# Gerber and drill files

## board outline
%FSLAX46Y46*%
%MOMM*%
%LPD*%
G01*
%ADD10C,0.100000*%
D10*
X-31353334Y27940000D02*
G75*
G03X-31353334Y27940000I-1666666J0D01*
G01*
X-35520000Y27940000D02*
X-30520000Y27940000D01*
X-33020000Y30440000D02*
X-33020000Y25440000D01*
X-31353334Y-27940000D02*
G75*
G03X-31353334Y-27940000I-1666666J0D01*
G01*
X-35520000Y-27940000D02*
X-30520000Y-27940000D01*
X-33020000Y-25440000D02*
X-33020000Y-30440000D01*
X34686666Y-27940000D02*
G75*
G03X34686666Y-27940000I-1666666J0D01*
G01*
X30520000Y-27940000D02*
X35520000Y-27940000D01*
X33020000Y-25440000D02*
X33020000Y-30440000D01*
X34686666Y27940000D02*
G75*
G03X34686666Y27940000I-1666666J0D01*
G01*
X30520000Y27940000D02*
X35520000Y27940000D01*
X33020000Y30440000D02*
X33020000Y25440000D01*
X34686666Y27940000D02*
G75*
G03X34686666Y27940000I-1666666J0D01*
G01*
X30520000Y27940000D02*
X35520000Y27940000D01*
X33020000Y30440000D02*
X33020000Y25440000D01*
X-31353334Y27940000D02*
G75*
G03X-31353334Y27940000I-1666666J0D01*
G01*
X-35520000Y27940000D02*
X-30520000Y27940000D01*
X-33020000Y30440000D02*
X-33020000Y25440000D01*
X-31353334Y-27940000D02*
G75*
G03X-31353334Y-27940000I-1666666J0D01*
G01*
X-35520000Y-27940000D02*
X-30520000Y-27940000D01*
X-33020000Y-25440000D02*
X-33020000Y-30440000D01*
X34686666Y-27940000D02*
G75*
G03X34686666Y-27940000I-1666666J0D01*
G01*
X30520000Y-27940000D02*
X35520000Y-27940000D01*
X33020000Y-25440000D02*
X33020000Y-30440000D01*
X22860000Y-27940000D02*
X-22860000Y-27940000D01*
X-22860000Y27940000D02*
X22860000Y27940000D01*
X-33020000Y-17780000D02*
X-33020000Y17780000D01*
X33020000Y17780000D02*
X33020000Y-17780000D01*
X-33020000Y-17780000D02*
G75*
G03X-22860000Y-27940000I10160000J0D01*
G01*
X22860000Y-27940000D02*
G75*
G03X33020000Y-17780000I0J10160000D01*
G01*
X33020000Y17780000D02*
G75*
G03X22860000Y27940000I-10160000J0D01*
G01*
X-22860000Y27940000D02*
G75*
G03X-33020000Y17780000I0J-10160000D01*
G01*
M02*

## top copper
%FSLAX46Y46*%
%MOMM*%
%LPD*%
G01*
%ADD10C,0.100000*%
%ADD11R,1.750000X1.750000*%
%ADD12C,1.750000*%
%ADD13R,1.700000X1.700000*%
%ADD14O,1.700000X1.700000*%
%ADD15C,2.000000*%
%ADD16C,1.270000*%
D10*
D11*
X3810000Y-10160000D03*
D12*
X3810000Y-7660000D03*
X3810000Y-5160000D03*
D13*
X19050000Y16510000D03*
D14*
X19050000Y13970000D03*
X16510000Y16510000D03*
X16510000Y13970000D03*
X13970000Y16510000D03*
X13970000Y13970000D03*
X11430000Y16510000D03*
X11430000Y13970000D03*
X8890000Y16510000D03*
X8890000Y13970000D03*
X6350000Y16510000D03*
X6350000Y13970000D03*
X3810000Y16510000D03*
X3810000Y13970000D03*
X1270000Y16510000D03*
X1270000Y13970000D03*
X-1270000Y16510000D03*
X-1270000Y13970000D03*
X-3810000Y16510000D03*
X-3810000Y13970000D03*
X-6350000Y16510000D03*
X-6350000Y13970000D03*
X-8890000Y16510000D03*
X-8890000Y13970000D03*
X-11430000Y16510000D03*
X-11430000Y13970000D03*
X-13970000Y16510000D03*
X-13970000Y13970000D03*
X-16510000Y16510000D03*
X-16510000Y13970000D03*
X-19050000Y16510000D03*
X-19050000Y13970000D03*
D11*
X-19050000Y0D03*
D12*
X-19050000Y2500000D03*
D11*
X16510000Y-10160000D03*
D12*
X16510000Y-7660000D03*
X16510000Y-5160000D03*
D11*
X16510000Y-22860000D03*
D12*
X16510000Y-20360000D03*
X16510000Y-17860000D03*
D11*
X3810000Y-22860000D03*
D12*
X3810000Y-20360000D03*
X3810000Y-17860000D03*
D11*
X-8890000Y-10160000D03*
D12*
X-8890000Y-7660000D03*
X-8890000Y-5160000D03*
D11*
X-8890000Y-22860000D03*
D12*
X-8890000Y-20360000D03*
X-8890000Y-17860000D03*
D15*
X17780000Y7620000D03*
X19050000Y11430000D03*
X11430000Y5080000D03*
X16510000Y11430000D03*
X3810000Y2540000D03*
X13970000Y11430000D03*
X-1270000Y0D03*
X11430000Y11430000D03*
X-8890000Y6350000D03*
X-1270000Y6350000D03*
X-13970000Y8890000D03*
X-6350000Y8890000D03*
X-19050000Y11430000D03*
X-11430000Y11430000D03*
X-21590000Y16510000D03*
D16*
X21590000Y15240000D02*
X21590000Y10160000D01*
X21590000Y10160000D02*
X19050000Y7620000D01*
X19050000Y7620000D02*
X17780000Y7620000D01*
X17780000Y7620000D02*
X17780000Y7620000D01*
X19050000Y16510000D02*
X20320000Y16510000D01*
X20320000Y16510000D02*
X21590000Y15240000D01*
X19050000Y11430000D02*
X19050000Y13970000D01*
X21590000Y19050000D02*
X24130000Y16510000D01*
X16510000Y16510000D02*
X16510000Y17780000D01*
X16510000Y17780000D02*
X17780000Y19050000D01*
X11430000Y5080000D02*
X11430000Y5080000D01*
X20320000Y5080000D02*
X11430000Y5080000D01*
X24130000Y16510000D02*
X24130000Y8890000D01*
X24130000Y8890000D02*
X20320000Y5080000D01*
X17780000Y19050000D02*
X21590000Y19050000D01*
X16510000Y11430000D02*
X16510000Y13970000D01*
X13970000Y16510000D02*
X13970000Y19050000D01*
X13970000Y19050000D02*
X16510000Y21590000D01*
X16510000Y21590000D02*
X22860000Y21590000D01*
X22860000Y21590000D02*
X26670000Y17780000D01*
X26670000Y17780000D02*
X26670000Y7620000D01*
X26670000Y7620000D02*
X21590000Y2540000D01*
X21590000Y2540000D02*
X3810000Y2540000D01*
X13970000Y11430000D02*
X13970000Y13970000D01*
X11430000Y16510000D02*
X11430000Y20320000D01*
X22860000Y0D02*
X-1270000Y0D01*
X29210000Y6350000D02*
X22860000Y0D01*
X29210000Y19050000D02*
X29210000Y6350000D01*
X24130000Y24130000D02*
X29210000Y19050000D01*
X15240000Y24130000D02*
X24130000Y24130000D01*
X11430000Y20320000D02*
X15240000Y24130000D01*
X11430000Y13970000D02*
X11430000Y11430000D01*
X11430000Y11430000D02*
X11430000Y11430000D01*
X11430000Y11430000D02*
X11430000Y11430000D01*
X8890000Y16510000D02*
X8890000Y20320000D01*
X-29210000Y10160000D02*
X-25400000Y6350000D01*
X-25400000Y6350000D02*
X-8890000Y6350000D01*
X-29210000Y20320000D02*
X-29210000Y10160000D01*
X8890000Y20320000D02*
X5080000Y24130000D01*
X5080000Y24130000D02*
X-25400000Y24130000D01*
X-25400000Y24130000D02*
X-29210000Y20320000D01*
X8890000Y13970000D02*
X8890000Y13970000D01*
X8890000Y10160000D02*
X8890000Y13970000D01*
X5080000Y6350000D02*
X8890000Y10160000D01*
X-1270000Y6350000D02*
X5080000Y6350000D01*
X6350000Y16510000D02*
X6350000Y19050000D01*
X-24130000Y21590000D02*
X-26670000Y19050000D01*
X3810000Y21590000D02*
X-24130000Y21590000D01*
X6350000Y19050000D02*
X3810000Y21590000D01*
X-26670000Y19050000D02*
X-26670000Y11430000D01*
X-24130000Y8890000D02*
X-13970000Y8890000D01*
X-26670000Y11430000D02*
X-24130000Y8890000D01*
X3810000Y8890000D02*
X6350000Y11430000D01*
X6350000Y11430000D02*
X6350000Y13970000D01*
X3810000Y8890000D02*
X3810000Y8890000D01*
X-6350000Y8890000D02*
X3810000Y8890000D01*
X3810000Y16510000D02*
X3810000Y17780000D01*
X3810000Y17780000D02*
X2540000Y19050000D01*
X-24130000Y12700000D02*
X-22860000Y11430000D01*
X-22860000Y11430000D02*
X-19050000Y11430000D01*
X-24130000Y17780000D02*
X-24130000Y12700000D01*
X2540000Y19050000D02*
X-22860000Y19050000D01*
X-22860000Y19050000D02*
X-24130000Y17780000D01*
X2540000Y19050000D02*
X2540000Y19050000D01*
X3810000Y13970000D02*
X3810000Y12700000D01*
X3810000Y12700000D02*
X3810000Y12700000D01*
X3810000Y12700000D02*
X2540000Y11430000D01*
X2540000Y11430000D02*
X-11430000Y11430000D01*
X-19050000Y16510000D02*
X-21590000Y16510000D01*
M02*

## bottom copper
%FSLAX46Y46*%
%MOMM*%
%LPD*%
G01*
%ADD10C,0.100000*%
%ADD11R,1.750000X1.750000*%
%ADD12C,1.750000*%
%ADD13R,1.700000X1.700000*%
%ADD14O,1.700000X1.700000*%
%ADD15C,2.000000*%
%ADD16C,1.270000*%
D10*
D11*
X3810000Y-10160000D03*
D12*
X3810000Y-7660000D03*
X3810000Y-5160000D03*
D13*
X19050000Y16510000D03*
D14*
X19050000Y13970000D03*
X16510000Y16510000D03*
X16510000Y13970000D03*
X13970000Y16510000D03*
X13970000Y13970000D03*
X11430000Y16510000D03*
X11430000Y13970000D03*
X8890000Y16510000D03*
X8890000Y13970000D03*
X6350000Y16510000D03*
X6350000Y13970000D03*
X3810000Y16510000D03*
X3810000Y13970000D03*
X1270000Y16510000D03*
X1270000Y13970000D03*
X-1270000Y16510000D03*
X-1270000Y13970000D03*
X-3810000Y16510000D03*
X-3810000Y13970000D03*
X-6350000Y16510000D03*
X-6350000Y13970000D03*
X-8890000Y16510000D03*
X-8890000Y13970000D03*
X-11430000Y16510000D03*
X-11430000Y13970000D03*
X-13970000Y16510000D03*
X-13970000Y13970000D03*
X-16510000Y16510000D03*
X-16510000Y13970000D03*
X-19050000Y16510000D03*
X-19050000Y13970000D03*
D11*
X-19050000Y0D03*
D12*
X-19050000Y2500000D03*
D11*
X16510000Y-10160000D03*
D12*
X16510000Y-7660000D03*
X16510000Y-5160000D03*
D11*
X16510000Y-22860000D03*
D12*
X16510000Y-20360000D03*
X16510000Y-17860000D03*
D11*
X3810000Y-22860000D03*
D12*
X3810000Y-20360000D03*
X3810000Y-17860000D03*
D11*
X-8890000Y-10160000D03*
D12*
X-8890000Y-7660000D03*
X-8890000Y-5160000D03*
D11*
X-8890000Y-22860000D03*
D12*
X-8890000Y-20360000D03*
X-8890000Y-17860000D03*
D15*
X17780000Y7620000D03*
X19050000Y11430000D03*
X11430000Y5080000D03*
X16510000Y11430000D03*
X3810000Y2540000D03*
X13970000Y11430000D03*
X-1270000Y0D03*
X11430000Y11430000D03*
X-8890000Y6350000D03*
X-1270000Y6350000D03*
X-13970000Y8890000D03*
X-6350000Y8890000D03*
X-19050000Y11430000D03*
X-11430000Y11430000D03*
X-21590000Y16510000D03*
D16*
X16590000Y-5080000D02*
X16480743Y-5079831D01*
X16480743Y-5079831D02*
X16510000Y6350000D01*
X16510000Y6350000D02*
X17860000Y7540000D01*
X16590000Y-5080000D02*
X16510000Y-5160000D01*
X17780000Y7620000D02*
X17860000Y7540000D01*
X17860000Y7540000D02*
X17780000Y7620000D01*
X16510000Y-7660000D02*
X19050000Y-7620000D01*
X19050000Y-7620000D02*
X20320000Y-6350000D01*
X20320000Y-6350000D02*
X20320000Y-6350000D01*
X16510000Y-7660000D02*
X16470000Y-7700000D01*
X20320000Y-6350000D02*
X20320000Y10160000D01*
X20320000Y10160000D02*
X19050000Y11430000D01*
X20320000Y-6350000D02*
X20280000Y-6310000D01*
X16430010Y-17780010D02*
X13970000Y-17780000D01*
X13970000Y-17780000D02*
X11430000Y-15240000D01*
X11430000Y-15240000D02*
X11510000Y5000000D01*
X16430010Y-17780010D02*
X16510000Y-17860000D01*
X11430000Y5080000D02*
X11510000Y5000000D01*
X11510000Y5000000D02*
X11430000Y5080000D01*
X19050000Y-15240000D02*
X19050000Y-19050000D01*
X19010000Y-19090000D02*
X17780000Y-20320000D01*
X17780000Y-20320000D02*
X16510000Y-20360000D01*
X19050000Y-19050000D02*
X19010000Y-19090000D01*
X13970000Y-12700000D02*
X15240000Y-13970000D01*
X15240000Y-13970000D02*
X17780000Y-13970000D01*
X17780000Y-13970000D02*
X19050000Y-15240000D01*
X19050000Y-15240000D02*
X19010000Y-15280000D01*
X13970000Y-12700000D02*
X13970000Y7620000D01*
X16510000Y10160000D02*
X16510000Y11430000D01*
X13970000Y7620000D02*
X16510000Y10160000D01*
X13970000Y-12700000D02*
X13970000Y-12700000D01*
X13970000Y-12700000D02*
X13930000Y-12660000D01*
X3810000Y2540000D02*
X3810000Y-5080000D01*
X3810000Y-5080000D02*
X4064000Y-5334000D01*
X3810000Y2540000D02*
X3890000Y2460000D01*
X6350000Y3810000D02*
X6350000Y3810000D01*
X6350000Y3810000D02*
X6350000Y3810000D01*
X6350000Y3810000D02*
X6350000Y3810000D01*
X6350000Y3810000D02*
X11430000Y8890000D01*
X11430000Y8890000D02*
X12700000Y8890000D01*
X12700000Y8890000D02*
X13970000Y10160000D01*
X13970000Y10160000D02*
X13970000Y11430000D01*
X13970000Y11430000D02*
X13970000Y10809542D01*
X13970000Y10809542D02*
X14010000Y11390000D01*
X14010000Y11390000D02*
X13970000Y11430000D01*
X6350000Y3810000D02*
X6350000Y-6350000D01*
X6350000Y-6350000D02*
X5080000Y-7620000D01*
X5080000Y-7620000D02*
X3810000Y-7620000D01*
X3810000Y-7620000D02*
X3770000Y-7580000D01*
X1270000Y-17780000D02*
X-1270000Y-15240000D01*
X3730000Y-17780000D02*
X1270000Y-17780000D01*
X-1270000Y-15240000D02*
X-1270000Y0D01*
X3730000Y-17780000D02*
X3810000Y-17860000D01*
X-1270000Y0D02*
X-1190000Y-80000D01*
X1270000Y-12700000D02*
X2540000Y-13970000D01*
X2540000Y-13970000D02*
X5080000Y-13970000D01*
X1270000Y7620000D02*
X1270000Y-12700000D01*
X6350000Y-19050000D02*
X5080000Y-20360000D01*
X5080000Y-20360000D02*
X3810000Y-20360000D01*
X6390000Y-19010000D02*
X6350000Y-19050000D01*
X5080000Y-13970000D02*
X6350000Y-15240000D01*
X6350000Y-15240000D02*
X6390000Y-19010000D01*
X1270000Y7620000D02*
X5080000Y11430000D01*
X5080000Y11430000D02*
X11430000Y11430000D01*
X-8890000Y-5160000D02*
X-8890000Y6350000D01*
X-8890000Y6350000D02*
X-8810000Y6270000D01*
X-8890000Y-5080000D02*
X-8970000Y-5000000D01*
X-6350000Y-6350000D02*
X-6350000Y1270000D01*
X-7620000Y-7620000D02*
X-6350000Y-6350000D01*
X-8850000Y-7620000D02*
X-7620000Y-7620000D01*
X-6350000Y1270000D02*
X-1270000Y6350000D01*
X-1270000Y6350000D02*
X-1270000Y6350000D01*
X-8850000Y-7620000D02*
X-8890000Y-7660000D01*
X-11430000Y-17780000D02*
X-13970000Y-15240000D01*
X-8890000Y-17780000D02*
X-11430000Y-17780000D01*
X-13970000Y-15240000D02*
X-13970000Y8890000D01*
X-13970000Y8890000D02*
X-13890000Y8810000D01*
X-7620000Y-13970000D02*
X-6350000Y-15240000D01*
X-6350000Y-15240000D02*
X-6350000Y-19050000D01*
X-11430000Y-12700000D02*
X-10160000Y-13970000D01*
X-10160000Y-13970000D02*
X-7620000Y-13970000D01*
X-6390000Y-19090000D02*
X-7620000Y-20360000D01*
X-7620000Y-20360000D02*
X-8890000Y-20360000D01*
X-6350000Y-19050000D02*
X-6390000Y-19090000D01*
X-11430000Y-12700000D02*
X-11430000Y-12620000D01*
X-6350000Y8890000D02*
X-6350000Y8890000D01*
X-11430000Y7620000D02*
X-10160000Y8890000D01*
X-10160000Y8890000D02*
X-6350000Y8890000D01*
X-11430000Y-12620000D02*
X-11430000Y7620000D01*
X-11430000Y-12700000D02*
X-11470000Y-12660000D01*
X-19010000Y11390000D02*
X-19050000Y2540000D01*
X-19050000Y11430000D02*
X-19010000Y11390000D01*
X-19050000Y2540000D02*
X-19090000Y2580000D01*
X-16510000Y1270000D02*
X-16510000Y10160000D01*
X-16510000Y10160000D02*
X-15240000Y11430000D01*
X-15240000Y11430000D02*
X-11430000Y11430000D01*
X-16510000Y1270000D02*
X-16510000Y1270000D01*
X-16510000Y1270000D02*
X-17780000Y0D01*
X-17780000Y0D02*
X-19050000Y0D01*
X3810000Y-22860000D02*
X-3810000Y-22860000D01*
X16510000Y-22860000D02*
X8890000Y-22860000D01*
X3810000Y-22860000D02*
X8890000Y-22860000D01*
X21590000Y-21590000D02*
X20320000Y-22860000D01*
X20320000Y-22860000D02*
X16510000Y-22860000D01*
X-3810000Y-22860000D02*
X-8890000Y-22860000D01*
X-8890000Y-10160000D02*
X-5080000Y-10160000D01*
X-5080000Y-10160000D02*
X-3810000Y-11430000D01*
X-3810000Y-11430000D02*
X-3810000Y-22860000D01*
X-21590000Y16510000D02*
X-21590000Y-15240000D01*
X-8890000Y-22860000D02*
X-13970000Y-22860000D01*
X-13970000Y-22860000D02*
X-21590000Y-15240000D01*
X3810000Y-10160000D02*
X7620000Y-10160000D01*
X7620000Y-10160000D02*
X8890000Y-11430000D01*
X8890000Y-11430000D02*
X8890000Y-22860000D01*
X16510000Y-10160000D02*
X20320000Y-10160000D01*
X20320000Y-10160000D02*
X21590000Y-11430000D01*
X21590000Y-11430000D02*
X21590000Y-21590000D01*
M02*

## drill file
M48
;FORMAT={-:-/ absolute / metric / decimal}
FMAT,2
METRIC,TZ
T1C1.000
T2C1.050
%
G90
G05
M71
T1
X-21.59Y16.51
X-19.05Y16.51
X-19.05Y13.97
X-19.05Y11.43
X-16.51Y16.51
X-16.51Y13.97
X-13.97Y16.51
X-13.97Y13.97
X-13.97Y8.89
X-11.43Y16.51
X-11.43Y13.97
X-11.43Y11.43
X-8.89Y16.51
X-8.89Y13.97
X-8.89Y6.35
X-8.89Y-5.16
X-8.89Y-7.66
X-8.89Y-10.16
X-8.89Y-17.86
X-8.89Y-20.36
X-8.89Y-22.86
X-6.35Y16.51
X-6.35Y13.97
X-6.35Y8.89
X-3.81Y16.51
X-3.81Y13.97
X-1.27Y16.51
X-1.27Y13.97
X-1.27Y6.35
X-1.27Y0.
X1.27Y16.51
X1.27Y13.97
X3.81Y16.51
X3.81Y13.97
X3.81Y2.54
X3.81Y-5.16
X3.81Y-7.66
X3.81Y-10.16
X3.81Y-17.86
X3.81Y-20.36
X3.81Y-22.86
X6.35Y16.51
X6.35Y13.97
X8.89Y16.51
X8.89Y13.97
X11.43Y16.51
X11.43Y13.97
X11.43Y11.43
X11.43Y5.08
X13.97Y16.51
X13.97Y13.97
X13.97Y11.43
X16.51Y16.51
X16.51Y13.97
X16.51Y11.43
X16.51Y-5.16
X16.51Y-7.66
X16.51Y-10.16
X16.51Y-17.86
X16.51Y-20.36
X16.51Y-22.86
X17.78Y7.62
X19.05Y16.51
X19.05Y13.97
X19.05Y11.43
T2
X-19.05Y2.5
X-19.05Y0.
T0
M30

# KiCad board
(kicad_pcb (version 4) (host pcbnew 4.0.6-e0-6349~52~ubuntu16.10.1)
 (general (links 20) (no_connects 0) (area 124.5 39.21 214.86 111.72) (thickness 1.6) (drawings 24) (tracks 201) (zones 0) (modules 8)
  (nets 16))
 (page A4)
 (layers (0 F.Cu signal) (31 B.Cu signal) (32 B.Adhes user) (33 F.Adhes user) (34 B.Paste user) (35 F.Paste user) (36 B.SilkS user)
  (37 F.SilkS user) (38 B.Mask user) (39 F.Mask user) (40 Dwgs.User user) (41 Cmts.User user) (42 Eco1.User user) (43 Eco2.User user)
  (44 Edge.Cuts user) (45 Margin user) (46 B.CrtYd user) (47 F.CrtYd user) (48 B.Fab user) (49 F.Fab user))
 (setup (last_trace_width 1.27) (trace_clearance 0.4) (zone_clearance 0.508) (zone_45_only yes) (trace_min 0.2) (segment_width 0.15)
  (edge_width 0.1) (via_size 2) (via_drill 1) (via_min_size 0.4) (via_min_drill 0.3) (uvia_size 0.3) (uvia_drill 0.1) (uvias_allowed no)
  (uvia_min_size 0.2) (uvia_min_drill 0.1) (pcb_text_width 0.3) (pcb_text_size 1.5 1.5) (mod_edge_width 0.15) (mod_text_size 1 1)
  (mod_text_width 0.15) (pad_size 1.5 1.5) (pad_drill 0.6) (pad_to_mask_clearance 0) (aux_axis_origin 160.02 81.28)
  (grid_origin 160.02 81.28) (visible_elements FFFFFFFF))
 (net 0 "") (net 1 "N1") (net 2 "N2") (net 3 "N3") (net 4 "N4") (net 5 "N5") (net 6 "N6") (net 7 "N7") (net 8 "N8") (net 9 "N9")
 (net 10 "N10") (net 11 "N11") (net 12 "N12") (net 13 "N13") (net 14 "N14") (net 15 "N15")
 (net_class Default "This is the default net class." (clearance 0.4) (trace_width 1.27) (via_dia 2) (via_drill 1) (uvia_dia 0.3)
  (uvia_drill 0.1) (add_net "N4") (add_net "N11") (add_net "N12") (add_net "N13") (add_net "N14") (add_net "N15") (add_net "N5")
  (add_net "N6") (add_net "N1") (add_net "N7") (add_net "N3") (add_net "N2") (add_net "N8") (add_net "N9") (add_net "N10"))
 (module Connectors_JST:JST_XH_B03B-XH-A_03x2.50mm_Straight (layer F.Cu) (at 163.83 91.44 90)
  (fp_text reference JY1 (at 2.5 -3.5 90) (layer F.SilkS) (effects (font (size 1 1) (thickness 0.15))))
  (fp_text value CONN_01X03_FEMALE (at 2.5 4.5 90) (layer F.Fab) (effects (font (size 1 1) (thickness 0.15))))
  (pad 1 thru_hole rect (at 0 0 90) (size 1.75 1.75) (drill 1) (layers *.Cu *.Mask) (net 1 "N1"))
  (pad 2 thru_hole circle (at 2.5 0 90) (size 1.75 1.75) (drill 1) (layers *.Cu *.Mask) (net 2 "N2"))
  (pad 3 thru_hole circle (at 5 0 90) (size 1.75 1.75) (drill 1) (layers *.Cu *.Mask) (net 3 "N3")))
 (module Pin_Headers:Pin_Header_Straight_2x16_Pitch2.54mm (layer F.Cu) (at 179.07 64.77 270)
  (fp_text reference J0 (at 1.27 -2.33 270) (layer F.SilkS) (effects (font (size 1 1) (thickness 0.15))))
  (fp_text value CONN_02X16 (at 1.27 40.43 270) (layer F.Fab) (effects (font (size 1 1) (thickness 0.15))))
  (pad 1 thru_hole rect (at 0 0 270) (size 1.7 1.7) (drill 1) (layers *.Cu *.Mask) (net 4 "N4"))
  (pad 2 thru_hole oval (at 2.54 0 270) (size 1.7 1.7) (drill 1) (layers *.Cu *.Mask) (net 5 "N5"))
  (pad 3 thru_hole oval (at 0 2.54 270) (size 1.7 1.7) (drill 1) (layers *.Cu *.Mask) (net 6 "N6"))
  (pad 4 thru_hole oval (at 2.54 2.54 270) (size 1.7 1.7) (drill 1) (layers *.Cu *.Mask) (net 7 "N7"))
  (pad 5 thru_hole oval (at 0 5.08 270) (size 1.7 1.7) (drill 1) (layers *.Cu *.Mask) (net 3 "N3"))
  (pad 6 thru_hole oval (at 2.54 5.08 270) (size 1.7 1.7) (drill 1) (layers *.Cu *.Mask) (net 2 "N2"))
  (pad 7 thru_hole oval (at 0 7.62 270) (size 1.7 1.7) (drill 1) (layers *.Cu *.Mask) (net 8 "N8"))
  (pad 8 thru_hole oval (at 2.54 7.62 270) (size 1.7 1.7) (drill 1) (layers *.Cu *.Mask) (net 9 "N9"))
  (pad 9 thru_hole oval (at 0 10.16 270) (size 1.7 1.7) (drill 1) (layers *.Cu *.Mask) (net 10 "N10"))
  (pad 10 thru_hole oval (at 2.54 10.16 270) (size 1.7 1.7) (drill 1) (layers *.Cu *.Mask) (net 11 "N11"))
  (pad 11 thru_hole oval (at 0 12.7 270) (size 1.7 1.7) (drill 1) (layers *.Cu *.Mask) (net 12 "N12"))
  (pad 12 thru_hole oval (at 2.54 12.7 270) (size 1.7 1.7) (drill 1) (layers *.Cu *.Mask) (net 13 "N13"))
  (pad 13 thru_hole oval (at 0 15.24 270) (size 1.7 1.7) (drill 1) (layers *.Cu *.Mask) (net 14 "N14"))
  (pad 14 thru_hole oval (at 2.54 15.24 270) (size 1.7 1.7) (drill 1) (layers *.Cu *.Mask) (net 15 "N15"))
  (pad 15 thru_hole oval (at 0 17.78 270) (size 1.7 1.7) (drill 1) (layers *.Cu *.Mask))
  (pad 16 thru_hole oval (at 2.54 17.78 270) (size 1.7 1.7) (drill 1) (layers *.Cu *.Mask))
  (pad 17 thru_hole oval (at 0 20.32 270) (size 1.7 1.7) (drill 1) (layers *.Cu *.Mask))
  (pad 18 thru_hole oval (at 2.54 20.32 270) (size 1.7 1.7) (drill 1) (layers *.Cu *.Mask))
  (pad 19 thru_hole oval (at 0 22.86 270) (size 1.7 1.7) (drill 1) (layers *.Cu *.Mask))
  (pad 20 thru_hole oval (at 2.54 22.86 270) (size 1.7 1.7) (drill 1) (layers *.Cu *.Mask))
  (pad 21 thru_hole oval (at 0 25.4 270) (size 1.7 1.7) (drill 1) (layers *.Cu *.Mask))
  (pad 22 thru_hole oval (at 2.54 25.4 270) (size 1.7 1.7) (drill 1) (layers *.Cu *.Mask))
  (pad 23 thru_hole oval (at 0 27.94 270) (size 1.7 1.7) (drill 1) (layers *.Cu *.Mask))
  (pad 24 thru_hole oval (at 2.54 27.94 270) (size 1.7 1.7) (drill 1) (layers *.Cu *.Mask))
  (pad 25 thru_hole oval (at 0 30.48 270) (size 1.7 1.7) (drill 1) (layers *.Cu *.Mask))
  (pad 26 thru_hole oval (at 2.54 30.48 270) (size 1.7 1.7) (drill 1) (layers *.Cu *.Mask))
  (pad 27 thru_hole oval (at 0 33.02 270) (size 1.7 1.7) (drill 1) (layers *.Cu *.Mask))
  (pad 28 thru_hole oval (at 2.54 33.02 270) (size 1.7 1.7) (drill 1) (layers *.Cu *.Mask))
  (pad 29 thru_hole oval (at 0 35.56 270) (size 1.7 1.7) (drill 1) (layers *.Cu *.Mask))
  (pad 30 thru_hole oval (at 2.54 35.56 270) (size 1.7 1.7) (drill 1) (layers *.Cu *.Mask))
  (pad 31 thru_hole oval (at 0 38.1 270) (size 1.7 1.7) (drill 1) (layers *.Cu *.Mask) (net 1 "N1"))
  (pad 32 thru_hole oval (at 2.54 38.1 270) (size 1.7 1.7) (drill 1) (layers *.Cu *.Mask)))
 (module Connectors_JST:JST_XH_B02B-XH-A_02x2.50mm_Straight (layer F.Cu) (at 140.97 81.28 90)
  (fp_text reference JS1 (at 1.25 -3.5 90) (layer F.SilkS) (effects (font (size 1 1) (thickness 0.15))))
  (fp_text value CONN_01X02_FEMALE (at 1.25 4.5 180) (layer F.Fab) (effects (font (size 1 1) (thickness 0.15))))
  (pad 1 thru_hole rect (at 0 0 90) (size 1.75 1.75) (drill 1.05) (layers *.Cu *.Mask) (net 15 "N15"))
  (pad 2 thru_hole circle (at 2.5 0 90) (size 1.75 1.75) (drill 1.05) (layers *.Cu *.Mask) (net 14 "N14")))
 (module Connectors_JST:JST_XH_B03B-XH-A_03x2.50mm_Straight (layer F.Cu) (at 176.53 91.44 90)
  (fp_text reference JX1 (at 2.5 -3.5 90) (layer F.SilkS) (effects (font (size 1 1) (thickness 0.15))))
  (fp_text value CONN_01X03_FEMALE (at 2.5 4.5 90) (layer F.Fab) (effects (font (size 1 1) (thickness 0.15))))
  (pad 1 thru_hole rect (at 0 0 90) (size 1.75 1.75) (drill 1) (layers *.Cu *.Mask) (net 1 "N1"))
  (pad 2 thru_hole circle (at 2.5 0 90) (size 1.75 1.75) (drill 1) (layers *.Cu *.Mask) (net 5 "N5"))
  (pad 3 thru_hole circle (at 5 0 90) (size 1.75 1.75) (drill 1) (layers *.Cu *.Mask) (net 4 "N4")))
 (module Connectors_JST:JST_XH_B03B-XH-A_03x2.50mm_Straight (layer F.Cu) (at 176.53 104.14 90)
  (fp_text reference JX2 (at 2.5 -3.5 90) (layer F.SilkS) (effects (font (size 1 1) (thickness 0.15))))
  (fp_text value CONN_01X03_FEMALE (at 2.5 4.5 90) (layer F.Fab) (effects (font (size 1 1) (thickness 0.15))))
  (pad 1 thru_hole rect (at 0 0 90) (size 1.75 1.75) (drill 1) (layers *.Cu *.Mask) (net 1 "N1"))
  (pad 2 thru_hole circle (at 2.5 0 90) (size 1.75 1.75) (drill 1) (layers *.Cu *.Mask) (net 7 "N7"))
  (pad 3 thru_hole circle (at 5 0 90) (size 1.75 1.75) (drill 1) (layers *.Cu *.Mask) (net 6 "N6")))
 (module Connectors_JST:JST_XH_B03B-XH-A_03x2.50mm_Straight (layer F.Cu) (at 163.83 104.14 90)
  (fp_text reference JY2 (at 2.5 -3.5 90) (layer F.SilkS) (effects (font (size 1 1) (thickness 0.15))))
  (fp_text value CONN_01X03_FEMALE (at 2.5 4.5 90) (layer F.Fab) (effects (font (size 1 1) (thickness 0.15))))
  (pad 1 thru_hole rect (at 0 0 90) (size 1.75 1.75) (drill 1) (layers *.Cu *.Mask) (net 1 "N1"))
  (pad 2 thru_hole circle (at 2.5 0 90) (size 1.75 1.75) (drill 1) (layers *.Cu *.Mask) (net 9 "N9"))
  (pad 3 thru_hole circle (at 5 0 90) (size 1.75 1.75) (drill 1) (layers *.Cu *.Mask) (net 8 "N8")))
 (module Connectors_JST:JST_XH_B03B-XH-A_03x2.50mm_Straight (layer F.Cu) (at 151.13 91.44 90)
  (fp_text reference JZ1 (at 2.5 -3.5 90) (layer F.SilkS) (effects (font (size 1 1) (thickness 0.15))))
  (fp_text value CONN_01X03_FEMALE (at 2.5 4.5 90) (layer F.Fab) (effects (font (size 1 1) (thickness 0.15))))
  (pad 1 thru_hole rect (at 0 0 90) (size 1.75 1.75) (drill 1) (layers *.Cu *.Mask) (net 1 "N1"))
  (pad 2 thru_hole circle (at 2.5 0 90) (size 1.75 1.75) (drill 1) (layers *.Cu *.Mask) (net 11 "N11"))
  (pad 3 thru_hole circle (at 5 0 90) (size 1.75 1.75) (drill 1) (layers *.Cu *.Mask) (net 10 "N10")))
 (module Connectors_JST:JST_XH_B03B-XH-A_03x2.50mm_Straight (layer F.Cu) (at 151.13 104.14 90)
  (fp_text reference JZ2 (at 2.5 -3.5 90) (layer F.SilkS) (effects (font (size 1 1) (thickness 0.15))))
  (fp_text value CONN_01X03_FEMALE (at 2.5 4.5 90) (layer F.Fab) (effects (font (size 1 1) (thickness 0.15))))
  (pad 1 thru_hole rect (at 0 0 90) (size 1.75 1.75) (drill 1) (layers *.Cu *.Mask) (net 1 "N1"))
  (pad 2 thru_hole circle (at 2.5 0 90) (size 1.75 1.75) (drill 1) (layers *.Cu *.Mask) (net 13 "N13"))
  (pad 3 thru_hole circle (at 5 0 90) (size 1.75 1.75) (drill 1) (layers *.Cu *.Mask) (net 12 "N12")))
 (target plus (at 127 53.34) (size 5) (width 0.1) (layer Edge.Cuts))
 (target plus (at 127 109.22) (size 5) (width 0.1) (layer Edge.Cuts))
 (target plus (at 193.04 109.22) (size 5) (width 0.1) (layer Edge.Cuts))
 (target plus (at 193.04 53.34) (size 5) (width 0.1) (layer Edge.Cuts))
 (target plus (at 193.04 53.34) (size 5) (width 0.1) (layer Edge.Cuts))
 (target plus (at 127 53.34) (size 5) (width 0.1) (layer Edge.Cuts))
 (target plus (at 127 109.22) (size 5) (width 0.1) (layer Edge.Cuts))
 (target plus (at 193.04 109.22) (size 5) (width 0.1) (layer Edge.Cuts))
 (gr_line (start 182.88 109.22) (end 137.16 109.22) (angle 90) (layer Edge.Cuts) (width 0.1))
 (gr_line (start 137.16 53.34) (end 182.88 53.34) (angle 90) (layer Edge.Cuts) (width 0.1))
 (gr_line (start 127 99.06) (end 127 63.5) (angle 90) (layer Edge.Cuts) (width 0.1))
 (gr_line (start 193.04 63.5) (end 193.04 99.06) (angle 90) (layer Edge.Cuts) (width 0.1))
 (gr_arc (start 137.16 99.06) (end 137.16 109.22) (angle 90) (layer Edge.Cuts) (width 0.1))
 (gr_arc (start 182.88 99.06) (end 193.04 99.06) (angle 90) (layer Edge.Cuts) (width 0.1))
 (gr_arc (start 182.88 63.5) (end 182.88 53.34) (angle 90) (layer Edge.Cuts) (width 0.1))
 (gr_arc (start 137.16 63.5) (end 127 63.5) (angle 90) (layer Edge.Cuts) (width 0.1))
 (segment (start 176.61 86.36) (end 176.500743 86.359831) (width 1.27) (layer B.Cu) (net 4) (status 30))
 (segment (start 176.500743 86.359831) (end 176.53 74.93) (width 1.27) (layer B.Cu) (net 4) (status 10))
 (segment (start 176.53 74.93) (end 177.88 73.74) (width 1.27) (layer B.Cu) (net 4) (status 10))
 (segment (start 176.61 86.36) (end 176.53 86.44) (width 1.27) (layer B.Cu) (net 4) (status 30))
 (via (at 177.8 73.66) (size 2) (drill 1) (layers F.Cu B.Cu) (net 4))
 (segment (start 181.61 66.04) (end 181.61 71.12) (width 1.27) (layer F.Cu) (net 4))
 (segment (start 181.61 71.12) (end 179.07 73.66) (width 1.27) (layer F.Cu) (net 4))
 (segment (start 179.07 73.66) (end 177.8 73.66) (width 1.27) (layer F.Cu) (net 4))
 (segment (start 177.8 73.66) (end 177.8 73.66) (width 1.27) (layer F.Cu) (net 4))
 (segment (start 179.07 64.77) (end 180.34 64.77) (width 1.27) (layer F.Cu) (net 4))
 (segment (start 180.34 64.77) (end 181.61 66.04) (width 1.27) (layer F.Cu) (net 4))
 (segment (start 177.8 73.66) (end 177.88 73.74) (width 1.27) (layer B.Cu) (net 4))
 (segment (start 177.88 73.74) (end 177.8 73.66) (width 1.27) (layer B.Cu) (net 4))
 (segment (start 176.53 88.94) (end 179.07 88.9) (width 1.27) (layer B.Cu) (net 5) (status 10))
 (segment (start 179.07 88.9) (end 180.34 87.63) (width 1.27) (layer B.Cu) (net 5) (status 10))
 (segment (start 180.34 87.63) (end 180.34 87.63) (width 1.27) (layer B.Cu) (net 5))
 (segment (start 176.53 88.94) (end 176.49 88.98) (width 1.27) (layer B.Cu) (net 5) (status 30))
 (segment (start 180.34 87.63) (end 180.34 71.12) (width 1.27) (layer B.Cu) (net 5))
 (segment (start 180.34 71.12) (end 179.07 69.85) (width 1.27) (layer B.Cu) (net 5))
 (via (at 179.07 69.85) (size 2) (drill 1) (layers F.Cu B.Cu) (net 5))
 (segment (start 179.07 69.85) (end 179.07 67.31) (width 1.27) (layer F.Cu) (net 5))
 (segment (start 180.34 87.63) (end 180.3 87.59) (width 1.27) (layer B.Cu) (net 5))
 (segment (start 181.61 62.23) (end 184.15 64.77) (width 1.27) (layer F.Cu) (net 6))
 (segment (start 176.45001 99.06001) (end 173.99 99.06) (width 1.27) (layer B.Cu) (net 6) (status 10))
 (segment (start 173.99 99.06) (end 171.45 96.52) (width 1.27) (layer B.Cu) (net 6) (status 10))
 (segment (start 171.45 96.52) (end 171.53 76.28) (width 1.27) (layer B.Cu) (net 6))
 (segment (start 176.45001 99.06001) (end 176.53 99.14) (width 1.27) (layer B.Cu) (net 6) (status 30))
 (segment (start 176.53 64.77) (end 176.53 63.5) (width 1.27) (layer F.Cu) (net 6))
 (segment (start 176.53 63.5) (end 177.8 62.23) (width 1.27) (layer F.Cu) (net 6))
 (via (at 171.45 76.2) (size 2) (drill 1) (layers F.Cu B.Cu) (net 6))
 (segment (start 171.45 76.2) (end 171.45 76.2) (width 1.27) (layer F.Cu) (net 6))
 (segment (start 180.34 76.2) (end 171.45 76.2) (width 1.27) (layer F.Cu) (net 6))
 (segment (start 184.15 64.77) (end 184.15 72.39) (width 1.27) (layer F.Cu) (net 6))
 (segment (start 184.15 72.39) (end 180.34 76.2) (width 1.27) (layer F.Cu) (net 6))
 (segment (start 177.8 62.23) (end 181.61 62.23) (width 1.27) (layer F.Cu) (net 6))
 (segment (start 171.45 76.2) (end 171.53 76.28) (width 1.27) (layer B.Cu) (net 6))
 (segment (start 171.53 76.28) (end 171.45 76.2) (width 1.27) (layer B.Cu) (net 6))
 (segment (start 179.07 96.52) (end 179.07 100.33) (width 1.27) (layer B.Cu) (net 7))
 (segment (start 179.03 100.37) (end 177.8 101.6) (width 1.27) (layer B.Cu) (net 7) (status 20))
 (segment (start 177.8 101.6) (end 176.53 101.64) (width 1.27) (layer B.Cu) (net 7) (status 20))
 (segment (start 179.07 100.33) (end 179.03 100.37) (width 1.27) (layer B.Cu) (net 7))
 (segment (start 173.99 93.98) (end 175.26 95.25) (width 1.27) (layer B.Cu) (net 7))
 (segment (start 175.26 95.25) (end 177.8 95.25) (width 1.27) (layer B.Cu) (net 7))
 (segment (start 177.8 95.25) (end 179.07 96.52) (width 1.27) (layer B.Cu) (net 7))
 (segment (start 179.07 96.52) (end 179.03 96.56) (width 1.27) (layer B.Cu) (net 7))
 (segment (start 173.99 93.98) (end 173.99 73.66) (width 1.27) (layer B.Cu) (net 7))
 (segment (start 176.53 69.85) (end 176.53 67.31) (width 1.27) (layer F.Cu) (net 7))
 (via (at 176.53 69.85) (size 2) (drill 1) (layers F.Cu B.Cu) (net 7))
 (segment (start 176.53 71.12) (end 176.53 69.85) (width 1.27) (layer B.Cu) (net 7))
 (segment (start 173.99 73.66) (end 176.53 71.12) (width 1.27) (layer B.Cu) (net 7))
 (segment (start 173.99 93.98) (end 173.99 93.98) (width 1.27) (layer B.Cu) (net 7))
 (segment (start 173.99 93.98) (end 173.95 93.94) (width 1.27) (layer B.Cu) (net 7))
 (segment (start 163.83 78.74) (end 163.83 86.36) (width 1.27) (layer B.Cu) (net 3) (status 20))
 (segment (start 163.83 86.36) (end 164.084 86.614) (width 1.27) (layer B.Cu) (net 3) (status 30))
 (segment (start 173.99 64.77) (end 173.99 62.23) (width 1.27) (layer F.Cu) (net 3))
 (segment (start 173.99 62.23) (end 176.53 59.69) (width 1.27) (layer F.Cu) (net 3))
 (segment (start 176.53 59.69) (end 182.88 59.69) (width 1.27) (layer F.Cu) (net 3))
 (segment (start 182.88 59.69) (end 186.69 63.5) (width 1.27) (layer F.Cu) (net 3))
 (segment (start 186.69 63.5) (end 186.69 73.66) (width 1.27) (layer F.Cu) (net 3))
 (segment (start 186.69 73.66) (end 181.61 78.74) (width 1.27) (layer F.Cu) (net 3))
 (segment (start 181.61 78.74) (end 163.83 78.74) (width 1.27) (layer F.Cu) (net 3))
 (via (at 163.83 78.74) (size 2) (drill 1) (layers F.Cu B.Cu) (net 3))
 (segment (start 163.83 78.74) (end 163.91 78.82) (width 1.27) (layer B.Cu) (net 3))
 (segment (start 166.37 77.47) (end 166.37 77.47) (width 1.27) (layer B.Cu) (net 2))
 (segment (start 166.37 77.47) (end 166.37 77.47) (width 1.27) (layer B.Cu) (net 2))
 (segment (start 166.37 77.47) (end 166.37 77.47) (width 1.27) (layer B.Cu) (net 2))
 (segment (start 166.37 77.47) (end 171.45 72.39) (width 1.27) (layer B.Cu) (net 2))
 (segment (start 171.45 72.39) (end 172.72 72.39) (width 1.27) (layer B.Cu) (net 2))
 (segment (start 172.72 72.39) (end 173.99 71.12) (width 1.27) (layer B.Cu) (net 2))
 (segment (start 173.99 71.12) (end 173.99 69.85) (width 1.27) (layer B.Cu) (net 2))
 (segment (start 173.99 69.85) (end 173.99 70.470458) (width 1.27) (layer B.Cu) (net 2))
 (segment (start 173.99 70.470458) (end 174.03 69.89) (width 1.27) (layer B.Cu) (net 2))
 (segment (start 173.99 69.85) (end 173.99 67.31) (width 1.27) (layer F.Cu) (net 2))
 (via (at 173.99 69.85) (size 2) (drill 1) (layers F.Cu B.Cu) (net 2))
 (segment (start 174.03 69.89) (end 173.99 69.85) (width 1.27) (layer B.Cu) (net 2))
 (segment (start 166.37 77.47) (end 166.37 87.63) (width 1.27) (layer B.Cu) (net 2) (status 20))
 (segment (start 166.37 87.63) (end 165.1 88.9) (width 1.27) (layer B.Cu) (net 2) (status 20))
 (segment (start 165.1 88.9) (end 163.83 88.9) (width 1.27) (layer B.Cu) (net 2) (status 20))
 (segment (start 163.83 88.9) (end 163.79 88.86) (width 1.27) (layer B.Cu) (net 2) (status 30))
 (segment (start 161.29 99.06) (end 158.75 96.52) (width 1.27) (layer B.Cu) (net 8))
 (segment (start 163.75 99.06) (end 161.29 99.06) (width 1.27) (layer B.Cu) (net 8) (status 10))
 (segment (start 158.75 96.52) (end 158.75 81.28) (width 1.27) (layer B.Cu) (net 8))
 (segment (start 163.75 99.06) (end 163.83 99.14) (width 1.27) (layer B.Cu) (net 8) (status 30))
 (segment (start 171.45 64.77) (end 171.45 60.96) (width 1.27) (layer F.Cu) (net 8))
 (via (at 158.75 81.28) (size 2) (drill 1) (layers F.Cu B.Cu) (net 8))
 (segment (start 182.88 81.28) (end 158.75 81.28) (width 1.27) (layer F.Cu) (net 8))
 (segment (start 189.23 74.93) (end 182.88 81.28) (width 1.27) (layer F.Cu) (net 8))
 (segment (start 189.23 62.23) (end 189.23 74.93) (width 1.27) (layer F.Cu) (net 8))
 (segment (start 184.15 57.15) (end 189.23 62.23) (width 1.27) (layer F.Cu) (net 8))
 (segment (start 175.26 57.15) (end 184.15 57.15) (width 1.27) (layer F.Cu) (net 8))
 (segment (start 171.45 60.96) (end 175.26 57.15) (width 1.27) (layer F.Cu) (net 8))
 (segment (start 158.75 81.28) (end 158.83 81.36) (width 1.27) (layer B.Cu) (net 8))
 (segment (start 171.45 67.31) (end 171.45 69.85) (width 1.27) (layer F.Cu) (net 9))
 (segment (start 161.29 93.98) (end 162.56 95.25) (width 1.27) (layer B.Cu) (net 9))
 (segment (start 162.56 95.25) (end 165.1 95.25) (width 1.27) (layer B.Cu) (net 9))
 (segment (start 161.29 73.66) (end 161.29 93.98) (width 1.27) (layer B.Cu) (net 9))
 (segment (start 166.37 100.33) (end 165.1 101.64) (width 1.27) (layer B.Cu) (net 9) (status 20))
 (segment (start 165.1 101.64) (end 163.83 101.64) (width 1.27) (layer B.Cu) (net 9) (status 20))
 (segment (start 166.41 100.29) (end 166.37 100.33) (width 1.27) (layer B.Cu) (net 9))
 (segment (start 165.1 95.25) (end 166.37 96.52) (width 1.27) (layer B.Cu) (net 9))
 (segment (start 166.37 96.52) (end 166.41 100.29) (width 1.27) (layer B.Cu) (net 9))
 (segment (start 171.45 69.85) (end 171.45 69.85) (width 1.27) (layer F.Cu) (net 9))
 (segment (start 171.45 69.85) (end 171.45 69.85) (width 1.27) (layer F.Cu) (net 9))
 (via (at 171.45 69.85) (size 2) (drill 1) (layers F.Cu B.Cu) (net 9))
 (segment (start 161.29 73.66) (end 165.1 69.85) (width 1.27) (layer B.Cu) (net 9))
 (segment (start 165.1 69.85) (end 171.45 69.85) (width 1.27) (layer B.Cu) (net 9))
 (segment (start 151.13 86.44) (end 151.13 74.93) (width 1.27) (layer B.Cu) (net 10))
 (segment (start 168.91 64.77) (end 168.91 60.96) (width 1.27) (layer F.Cu) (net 10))
 (segment (start 151.13 74.93) (end 151.21 75.01) (width 1.27) (layer B.Cu) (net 10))
 (via (at 151.13 74.93) (size 2) (drill 1) (layers F.Cu B.Cu) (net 10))
 (segment (start 130.81 71.12) (end 134.62 74.93) (width 1.27) (layer F.Cu) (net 10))
 (segment (start 134.62 74.93) (end 151.13 74.93) (width 1.27) (layer F.Cu) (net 10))
 (segment (start 130.81 60.96) (end 130.81 71.12) (width 1.27) (layer F.Cu) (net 10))
 (segment (start 168.91 60.96) (end 165.1 57.15) (width 1.27) (layer F.Cu) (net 10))
 (segment (start 165.1 57.15) (end 134.62 57.15) (width 1.27) (layer F.Cu) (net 10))
 (segment (start 134.62 57.15) (end 130.81 60.96) (width 1.27) (layer F.Cu) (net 10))
 (segment (start 151.13 86.36) (end 151.05 86.28) (width 1.27) (layer B.Cu) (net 10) (status 30))
 (segment (start 153.67 87.63) (end 153.67 80.01) (width 1.27) (layer B.Cu) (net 11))
 (segment (start 152.4 88.9) (end 153.67 87.63) (width 1.27) (layer B.Cu) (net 11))
 (segment (start 151.17 88.9) (end 152.4 88.9) (width 1.27) (layer B.Cu) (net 11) (status 10))
 (segment (start 153.67 80.01) (end 158.75 74.93) (width 1.27) (layer B.Cu) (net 11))
 (segment (start 168.91 67.31) (end 168.91 67.31) (width 1.27) (layer F.Cu) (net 11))
 (segment (start 168.91 71.12) (end 168.91 67.31) (width 1.27) (layer F.Cu) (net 11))
 (via (at 158.75 74.93) (size 2) (drill 1) (layers F.Cu B.Cu) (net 11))
 (segment (start 165.1 74.93) (end 168.91 71.12) (width 1.27) (layer F.Cu) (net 11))
 (segment (start 158.75 74.93) (end 165.1 74.93) (width 1.27) (layer F.Cu) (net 11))
 (segment (start 158.75 74.93) (end 158.75 74.93) (width 1.27) (layer B.Cu) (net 11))
 (segment (start 151.17 88.9) (end 151.13 88.94) (width 1.27) (layer B.Cu) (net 11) (status 30))
 (segment (start 148.59 99.06) (end 146.05 96.52) (width 1.27) (layer B.Cu) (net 12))
 (segment (start 151.13 99.06) (end 148.59 99.06) (width 1.27) (layer B.Cu) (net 12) (status 10))
 (segment (start 146.05 96.52) (end 146.05 72.39) (width 1.27) (layer B.Cu) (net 12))
 (segment (start 166.37 64.77) (end 166.37 62.23) (width 1.27) (layer F.Cu) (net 12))
 (segment (start 135.89 59.69) (end 133.35 62.23) (width 1.27) (layer F.Cu) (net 12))
 (segment (start 163.83 59.69) (end 135.89 59.69) (width 1.27) (layer F.Cu) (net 12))
 (segment (start 166.37 62.23) (end 163.83 59.69) (width 1.27) (layer F.Cu) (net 12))
 (segment (start 133.35 62.23) (end 133.35 69.85) (width 1.27) (layer F.Cu) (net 12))
 (segment (start 135.89 72.39) (end 146.05 72.39) (width 1.27) (layer F.Cu) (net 12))
 (segment (start 133.35 69.85) (end 135.89 72.39) (width 1.27) (layer F.Cu) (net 12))
 (via (at 146.05 72.39) (size 2) (drill 1) (layers F.Cu B.Cu) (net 12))
 (segment (start 146.05 72.39) (end 146.13 72.47) (width 1.27) (layer B.Cu) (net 12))
 (segment (start 163.83 72.39) (end 166.37 69.85) (width 1.27) (layer F.Cu) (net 13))
 (segment (start 166.37 69.85) (end 166.37 67.31) (width 1.27) (layer F.Cu) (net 13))
 (segment (start 163.83 72.39) (end 163.83 72.39) (width 1.27) (layer F.Cu) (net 13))
 (via (at 153.67 72.39) (size 2) (drill 1) (layers F.Cu B.Cu) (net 13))
 (segment (start 153.67 72.39) (end 163.83 72.39) (width 1.27) (layer F.Cu) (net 13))
 (segment (start 152.4 95.25) (end 153.67 96.52) (width 1.27) (layer B.Cu) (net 13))
 (segment (start 153.67 96.52) (end 153.67 100.33) (width 1.27) (layer B.Cu) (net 13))
 (segment (start 148.59 93.98) (end 149.86 95.25) (width 1.27) (layer B.Cu) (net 13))
 (segment (start 149.86 95.25) (end 152.4 95.25) (width 1.27) (layer B.Cu) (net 13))
 (segment (start 153.63 100.37) (end 152.4 101.64) (width 1.27) (layer B.Cu) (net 13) (status 20))
 (segment (start 152.4 101.64) (end 151.13 101.64) (width 1.27) (layer B.Cu) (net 13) (status 20))
 (segment (start 153.67 100.33) (end 153.63 100.37) (width 1.27) (layer B.Cu) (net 13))
 (segment (start 148.59 93.98) (end 148.59 93.9) (width 1.27) (layer B.Cu) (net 13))
 (segment (start 153.67 72.39) (end 153.67 72.39) (width 1.27) (layer B.Cu) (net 13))
 (segment (start 148.59 73.66) (end 149.86 72.39) (width 1.27) (layer B.Cu) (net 13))
 (segment (start 149.86 72.39) (end 153.67 72.39) (width 1.27) (layer B.Cu) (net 13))
 (segment (start 148.59 93.9) (end 148.59 73.66) (width 1.27) (layer B.Cu) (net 13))
 (segment (start 148.59 93.98) (end 148.55 93.94) (width 1.27) (layer B.Cu) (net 13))
 (segment (start 163.83 64.77) (end 163.83 63.5) (width 1.27) (layer F.Cu) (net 14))
 (segment (start 163.83 63.5) (end 162.56 62.23) (width 1.27) (layer F.Cu) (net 14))
 (segment (start 141.01 69.89) (end 140.97 78.74) (width 1.27) (layer B.Cu) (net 14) (status 20))
 (segment (start 140.97 69.85) (end 141.01 69.89) (width 1.27) (layer B.Cu) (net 14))
 (via (at 140.97 69.85) (size 2) (drill 1) (layers F.Cu B.Cu) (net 14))
 (segment (start 135.89 68.58) (end 137.16 69.85) (width 1.27) (layer F.Cu) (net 14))
 (segment (start 137.16 69.85) (end 140.97 69.85) (width 1.27) (layer F.Cu) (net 14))
 (segment (start 135.89 63.5) (end 135.89 68.58) (width 1.27) (layer F.Cu) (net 14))
 (segment (start 162.56 62.23) (end 137.16 62.23) (width 1.27) (layer F.Cu) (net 14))
 (segment (start 137.16 62.23) (end 135.89 63.5) (width 1.27) (layer F.Cu) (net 14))
 (segment (start 162.56 62.23) (end 162.56 62.23) (width 1.27) (layer F.Cu) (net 14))
 (segment (start 140.97 78.74) (end 140.93 78.7) (width 1.27) (layer B.Cu) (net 14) (status 30))
 (segment (start 163.83 67.31) (end 163.83 68.58) (width 1.27) (layer F.Cu) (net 15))
 (segment (start 163.83 68.58) (end 163.83 68.58) (width 1.27) (layer F.Cu) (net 15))
 (segment (start 163.83 68.58) (end 162.56 69.85) (width 1.27) (layer F.Cu) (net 15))
 (segment (start 162.56 69.85) (end 148.59 69.85) (width 1.27) (layer F.Cu) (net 15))
 (segment (start 143.51 80.01) (end 143.51 71.12) (width 1.27) (layer B.Cu) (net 15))
 (segment (start 143.51 71.12) (end 144.78 69.85) (width 1.27) (layer B.Cu) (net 15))
 (segment (start 144.78 69.85) (end 148.59 69.85) (width 1.27) (layer B.Cu) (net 15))
 (via (at 148.59 69.85) (size 2) (drill 1) (layers F.Cu B.Cu) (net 15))
 (segment (start 143.51 80.01) (end 143.51 80.01) (width 1.27) (layer B.Cu) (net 15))
 (segment (start 143.51 80.01) (end 142.24 81.28) (width 1.27) (layer B.Cu) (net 15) (status 20))
 (segment (start 142.24 81.28) (end 140.97 81.28) (width 1.27) (layer B.Cu) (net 15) (status 20))
 (segment (start 163.83 104.14) (end 156.21 104.14) (width 1.27) (layer B.Cu) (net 1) (status 10))
 (segment (start 176.53 104.14) (end 168.91 104.14) (width 1.27) (layer B.Cu) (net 1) (status 10))
 (segment (start 163.83 104.14) (end 168.91 104.14) (width 1.27) (layer B.Cu) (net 1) (status 10))
 (segment (start 181.61 102.87) (end 180.34 104.14) (width 1.27) (layer B.Cu) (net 1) (status 20))
 (segment (start 180.34 104.14) (end 176.53 104.14) (width 1.27) (layer B.Cu) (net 1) (status 20))
 (segment (start 156.21 104.14) (end 151.13 104.14) (width 1.27) (layer B.Cu) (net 1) (status 20))
 (segment (start 151.13 91.44) (end 154.94 91.44) (width 1.27) (layer B.Cu) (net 1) (status 10))
 (segment (start 154.94 91.44) (end 156.21 92.71) (width 1.27) (layer B.Cu) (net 1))
 (segment (start 156.21 92.71) (end 156.21 104.14) (width 1.27) (layer B.Cu) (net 1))
 (segment (start 138.43 64.77) (end 138.43 96.52) (width 1.27) (layer B.Cu) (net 1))
 (via (at 138.43 64.77) (size 2) (drill 1) (layers F.Cu B.Cu) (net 1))
 (segment (start 140.97 64.77) (end 138.43 64.77) (width 1.27) (layer F.Cu) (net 1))
 (segment (start 151.13 104.14) (end 146.05 104.14) (width 1.27) (layer B.Cu) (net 1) (status 10))
 (segment (start 146.05 104.14) (end 138.43 96.52) (width 1.27) (layer B.Cu) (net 1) (status 10))
 (segment (start 163.83 91.44) (end 167.64 91.44) (width 1.27) (layer B.Cu) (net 1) (status 10))
 (segment (start 167.64 91.44) (end 168.91 92.71) (width 1.27) (layer B.Cu) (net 1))
 (segment (start 168.91 92.71) (end 168.91 104.14) (width 1.27) (layer B.Cu) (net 1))
 (segment (start 176.53 91.44) (end 180.34 91.44) (width 1.27) (layer B.Cu) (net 1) (status 10))
 (segment (start 180.34 91.44) (end 181.61 92.71) (width 1.27) (layer B.Cu) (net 1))
 (segment (start 181.61 92.71) (end 181.61 102.87) (width 1.27) (layer B.Cu) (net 1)))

